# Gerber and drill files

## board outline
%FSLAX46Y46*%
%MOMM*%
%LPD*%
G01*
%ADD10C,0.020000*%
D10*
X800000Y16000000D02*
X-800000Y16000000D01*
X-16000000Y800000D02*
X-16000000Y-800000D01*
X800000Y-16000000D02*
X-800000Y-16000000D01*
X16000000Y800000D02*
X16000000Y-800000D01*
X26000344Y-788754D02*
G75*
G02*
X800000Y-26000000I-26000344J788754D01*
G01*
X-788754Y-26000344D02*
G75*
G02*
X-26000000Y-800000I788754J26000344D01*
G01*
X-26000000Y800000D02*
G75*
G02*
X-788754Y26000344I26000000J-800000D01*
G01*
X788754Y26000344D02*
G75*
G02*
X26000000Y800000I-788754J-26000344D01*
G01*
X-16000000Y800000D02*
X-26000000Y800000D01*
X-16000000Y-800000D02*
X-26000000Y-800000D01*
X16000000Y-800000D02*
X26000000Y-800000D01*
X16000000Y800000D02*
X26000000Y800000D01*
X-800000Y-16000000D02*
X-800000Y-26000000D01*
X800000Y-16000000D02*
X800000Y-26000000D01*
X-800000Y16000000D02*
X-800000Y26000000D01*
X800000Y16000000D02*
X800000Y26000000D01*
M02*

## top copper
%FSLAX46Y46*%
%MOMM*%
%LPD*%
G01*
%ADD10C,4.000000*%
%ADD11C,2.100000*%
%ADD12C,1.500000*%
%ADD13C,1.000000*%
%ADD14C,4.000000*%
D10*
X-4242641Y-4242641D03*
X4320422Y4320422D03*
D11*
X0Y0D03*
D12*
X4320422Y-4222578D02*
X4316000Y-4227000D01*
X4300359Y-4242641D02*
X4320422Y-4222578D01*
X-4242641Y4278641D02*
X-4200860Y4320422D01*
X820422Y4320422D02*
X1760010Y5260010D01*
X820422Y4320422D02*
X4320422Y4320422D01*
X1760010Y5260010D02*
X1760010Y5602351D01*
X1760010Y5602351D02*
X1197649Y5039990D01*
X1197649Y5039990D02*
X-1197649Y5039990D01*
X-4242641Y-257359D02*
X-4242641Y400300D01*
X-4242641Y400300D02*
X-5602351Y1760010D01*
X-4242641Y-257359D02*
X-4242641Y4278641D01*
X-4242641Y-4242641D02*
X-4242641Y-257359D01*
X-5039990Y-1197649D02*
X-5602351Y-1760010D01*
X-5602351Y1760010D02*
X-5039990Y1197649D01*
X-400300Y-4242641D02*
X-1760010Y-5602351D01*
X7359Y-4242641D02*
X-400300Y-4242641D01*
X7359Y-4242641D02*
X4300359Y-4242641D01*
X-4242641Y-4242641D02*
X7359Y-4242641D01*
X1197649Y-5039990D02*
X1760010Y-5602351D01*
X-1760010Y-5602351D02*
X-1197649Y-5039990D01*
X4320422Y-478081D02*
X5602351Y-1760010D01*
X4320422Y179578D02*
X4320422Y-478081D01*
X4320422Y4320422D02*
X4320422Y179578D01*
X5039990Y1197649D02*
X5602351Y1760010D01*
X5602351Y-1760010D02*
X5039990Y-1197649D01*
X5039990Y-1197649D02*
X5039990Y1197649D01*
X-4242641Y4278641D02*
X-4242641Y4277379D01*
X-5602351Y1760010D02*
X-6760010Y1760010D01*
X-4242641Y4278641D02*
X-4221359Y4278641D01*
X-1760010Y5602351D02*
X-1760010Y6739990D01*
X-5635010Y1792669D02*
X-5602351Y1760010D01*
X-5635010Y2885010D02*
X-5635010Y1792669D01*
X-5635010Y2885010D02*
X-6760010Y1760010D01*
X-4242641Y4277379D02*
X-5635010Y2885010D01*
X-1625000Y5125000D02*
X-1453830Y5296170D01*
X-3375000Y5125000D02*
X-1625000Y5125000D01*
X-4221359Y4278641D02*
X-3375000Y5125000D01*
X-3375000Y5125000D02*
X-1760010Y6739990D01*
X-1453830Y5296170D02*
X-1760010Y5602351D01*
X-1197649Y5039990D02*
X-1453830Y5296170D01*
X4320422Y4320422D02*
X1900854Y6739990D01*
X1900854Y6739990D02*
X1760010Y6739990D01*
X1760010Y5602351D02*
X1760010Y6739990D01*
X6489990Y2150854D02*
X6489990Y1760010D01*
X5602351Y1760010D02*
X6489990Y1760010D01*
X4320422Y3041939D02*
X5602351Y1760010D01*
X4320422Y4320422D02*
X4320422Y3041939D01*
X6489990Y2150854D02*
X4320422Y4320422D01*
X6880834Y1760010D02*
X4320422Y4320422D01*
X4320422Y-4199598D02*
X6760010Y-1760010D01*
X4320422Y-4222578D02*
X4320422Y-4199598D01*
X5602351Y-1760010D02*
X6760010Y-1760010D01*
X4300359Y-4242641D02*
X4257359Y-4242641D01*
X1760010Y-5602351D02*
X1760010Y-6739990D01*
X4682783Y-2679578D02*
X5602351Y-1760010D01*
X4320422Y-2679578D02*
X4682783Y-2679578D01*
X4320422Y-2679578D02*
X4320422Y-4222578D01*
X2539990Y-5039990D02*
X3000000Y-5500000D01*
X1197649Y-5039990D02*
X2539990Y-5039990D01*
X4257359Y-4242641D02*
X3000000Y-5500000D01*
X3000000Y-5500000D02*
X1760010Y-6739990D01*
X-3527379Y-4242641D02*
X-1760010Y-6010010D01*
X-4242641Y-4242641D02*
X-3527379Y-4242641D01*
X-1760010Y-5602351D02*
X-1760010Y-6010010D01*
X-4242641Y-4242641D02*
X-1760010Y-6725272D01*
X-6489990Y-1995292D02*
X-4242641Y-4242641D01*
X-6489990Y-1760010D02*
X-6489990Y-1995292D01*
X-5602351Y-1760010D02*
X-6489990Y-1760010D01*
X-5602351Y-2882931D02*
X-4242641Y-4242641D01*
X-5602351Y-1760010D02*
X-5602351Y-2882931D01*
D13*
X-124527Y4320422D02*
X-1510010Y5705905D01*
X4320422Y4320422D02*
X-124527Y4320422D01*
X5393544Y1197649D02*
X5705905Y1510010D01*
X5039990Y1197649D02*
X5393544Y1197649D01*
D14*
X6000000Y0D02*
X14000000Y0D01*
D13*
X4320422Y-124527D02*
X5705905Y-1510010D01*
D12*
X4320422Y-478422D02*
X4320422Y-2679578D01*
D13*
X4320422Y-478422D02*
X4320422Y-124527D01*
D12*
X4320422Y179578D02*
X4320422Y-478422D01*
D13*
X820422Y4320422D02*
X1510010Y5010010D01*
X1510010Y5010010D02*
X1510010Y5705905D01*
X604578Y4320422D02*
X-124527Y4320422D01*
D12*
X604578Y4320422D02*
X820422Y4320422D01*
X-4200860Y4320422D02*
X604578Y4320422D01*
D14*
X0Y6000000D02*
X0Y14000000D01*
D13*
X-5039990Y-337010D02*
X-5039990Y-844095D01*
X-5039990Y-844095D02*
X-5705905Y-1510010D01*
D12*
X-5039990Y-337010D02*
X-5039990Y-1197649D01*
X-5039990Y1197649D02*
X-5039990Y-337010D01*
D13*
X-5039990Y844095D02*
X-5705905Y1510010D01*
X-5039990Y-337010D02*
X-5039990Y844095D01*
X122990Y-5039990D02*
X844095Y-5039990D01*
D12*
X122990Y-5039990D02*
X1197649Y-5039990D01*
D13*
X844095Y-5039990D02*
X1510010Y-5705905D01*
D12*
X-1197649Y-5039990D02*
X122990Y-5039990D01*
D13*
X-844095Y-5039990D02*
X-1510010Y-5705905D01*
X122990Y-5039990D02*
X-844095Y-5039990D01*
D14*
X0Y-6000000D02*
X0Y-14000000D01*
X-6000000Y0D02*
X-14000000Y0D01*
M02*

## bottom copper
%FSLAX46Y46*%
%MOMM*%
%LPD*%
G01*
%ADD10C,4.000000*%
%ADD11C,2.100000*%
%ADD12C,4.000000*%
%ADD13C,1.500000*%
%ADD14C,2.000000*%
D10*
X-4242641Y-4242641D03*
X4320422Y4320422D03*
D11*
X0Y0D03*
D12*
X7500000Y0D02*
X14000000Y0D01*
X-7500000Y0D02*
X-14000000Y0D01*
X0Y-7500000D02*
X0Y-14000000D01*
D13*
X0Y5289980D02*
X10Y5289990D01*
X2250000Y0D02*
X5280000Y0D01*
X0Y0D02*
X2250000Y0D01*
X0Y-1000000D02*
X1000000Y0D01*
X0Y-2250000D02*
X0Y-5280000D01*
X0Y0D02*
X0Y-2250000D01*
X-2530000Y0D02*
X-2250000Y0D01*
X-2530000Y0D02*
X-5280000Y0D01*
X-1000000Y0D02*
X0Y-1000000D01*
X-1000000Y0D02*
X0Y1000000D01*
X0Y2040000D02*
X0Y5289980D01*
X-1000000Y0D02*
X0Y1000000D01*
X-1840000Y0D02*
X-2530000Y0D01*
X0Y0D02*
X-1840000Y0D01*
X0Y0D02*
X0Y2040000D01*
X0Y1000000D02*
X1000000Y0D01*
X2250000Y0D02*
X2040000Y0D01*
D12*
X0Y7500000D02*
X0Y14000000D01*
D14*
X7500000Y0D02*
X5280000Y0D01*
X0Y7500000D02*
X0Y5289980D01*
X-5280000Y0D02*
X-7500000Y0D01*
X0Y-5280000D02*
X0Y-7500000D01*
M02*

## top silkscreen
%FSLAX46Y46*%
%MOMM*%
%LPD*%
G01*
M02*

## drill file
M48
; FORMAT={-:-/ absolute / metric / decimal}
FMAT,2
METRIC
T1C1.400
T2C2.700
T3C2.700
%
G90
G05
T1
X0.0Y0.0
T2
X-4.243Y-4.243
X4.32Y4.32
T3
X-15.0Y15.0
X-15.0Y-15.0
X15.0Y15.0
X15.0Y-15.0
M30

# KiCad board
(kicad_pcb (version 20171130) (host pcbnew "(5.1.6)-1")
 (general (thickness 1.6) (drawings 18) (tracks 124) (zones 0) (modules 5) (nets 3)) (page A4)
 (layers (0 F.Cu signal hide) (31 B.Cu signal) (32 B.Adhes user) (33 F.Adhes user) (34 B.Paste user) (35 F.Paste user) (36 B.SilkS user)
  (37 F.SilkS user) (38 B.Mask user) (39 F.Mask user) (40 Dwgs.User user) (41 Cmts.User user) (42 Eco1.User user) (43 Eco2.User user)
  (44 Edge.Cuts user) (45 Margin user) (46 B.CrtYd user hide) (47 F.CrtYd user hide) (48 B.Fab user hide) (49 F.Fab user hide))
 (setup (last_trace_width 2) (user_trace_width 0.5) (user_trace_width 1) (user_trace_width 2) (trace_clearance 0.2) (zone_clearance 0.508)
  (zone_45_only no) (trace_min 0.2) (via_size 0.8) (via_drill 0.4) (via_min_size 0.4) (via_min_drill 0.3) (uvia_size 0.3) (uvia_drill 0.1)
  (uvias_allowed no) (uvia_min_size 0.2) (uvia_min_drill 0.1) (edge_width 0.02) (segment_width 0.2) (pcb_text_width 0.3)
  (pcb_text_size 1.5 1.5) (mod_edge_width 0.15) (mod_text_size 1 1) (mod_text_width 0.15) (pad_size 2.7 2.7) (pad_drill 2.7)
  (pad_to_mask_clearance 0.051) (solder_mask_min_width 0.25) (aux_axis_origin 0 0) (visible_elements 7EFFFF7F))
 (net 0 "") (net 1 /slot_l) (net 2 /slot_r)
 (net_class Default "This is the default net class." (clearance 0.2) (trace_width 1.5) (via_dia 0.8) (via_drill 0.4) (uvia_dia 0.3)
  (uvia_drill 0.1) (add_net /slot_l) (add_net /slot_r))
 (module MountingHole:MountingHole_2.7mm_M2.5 (layer F.Cu) (at -15 -15 90)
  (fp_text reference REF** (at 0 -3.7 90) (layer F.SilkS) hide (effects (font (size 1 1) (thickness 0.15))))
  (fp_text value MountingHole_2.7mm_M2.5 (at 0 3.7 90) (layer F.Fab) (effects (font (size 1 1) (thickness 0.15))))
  (pad 1 np_thru_hole circle (at 0 0 90) (size 2.7 2.7) (drill 2.7) (layers *.Cu *.Mask)))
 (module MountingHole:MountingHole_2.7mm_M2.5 (layer F.Cu) (at 15 -15)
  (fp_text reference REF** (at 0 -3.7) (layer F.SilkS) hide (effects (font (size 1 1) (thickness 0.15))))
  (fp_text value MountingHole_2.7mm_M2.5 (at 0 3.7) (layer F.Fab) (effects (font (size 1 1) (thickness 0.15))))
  (pad 1 np_thru_hole circle (at 0 0) (size 2.7 2.7) (drill 2.7) (layers *.Cu *.Mask)))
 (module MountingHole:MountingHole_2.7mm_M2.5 (layer F.Cu) (at 15 15)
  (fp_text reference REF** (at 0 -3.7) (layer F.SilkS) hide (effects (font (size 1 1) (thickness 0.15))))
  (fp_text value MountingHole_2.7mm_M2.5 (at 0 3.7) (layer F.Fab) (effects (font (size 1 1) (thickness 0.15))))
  (pad 1 np_thru_hole circle (at 0 0) (size 2.7 2.7) (drill 2.7) (layers *.Cu *.Mask)))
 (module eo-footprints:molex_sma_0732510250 (layer F.Cu) (at 0 0 45)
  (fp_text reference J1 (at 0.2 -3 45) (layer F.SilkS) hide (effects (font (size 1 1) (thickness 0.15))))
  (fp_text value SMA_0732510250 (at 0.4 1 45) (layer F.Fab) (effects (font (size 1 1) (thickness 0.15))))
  (pad 2 thru_hole circle (at -6 0 45) (size 4 4) (drill 2.7) (layers *.Cu *.Mask) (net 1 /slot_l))
  (pad 2 thru_hole circle (at 6.11 0 45) (size 4 4) (drill 2.7) (layers *.Cu *.Mask) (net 1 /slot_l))
  (pad 1 thru_hole circle (at 0 0 45) (size 2.1 2.1) (drill 1.4) (layers *.Cu *.Mask) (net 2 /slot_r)))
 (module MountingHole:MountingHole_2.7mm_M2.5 (layer F.Cu) (at -15 15)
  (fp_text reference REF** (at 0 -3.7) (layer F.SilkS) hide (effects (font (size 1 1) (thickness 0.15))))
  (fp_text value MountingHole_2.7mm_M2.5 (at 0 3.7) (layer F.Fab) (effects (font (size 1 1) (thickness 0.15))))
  (pad 1 np_thru_hole circle (at 0 0) (size 2.7 2.7) (drill 2.7) (layers *.Cu *.Mask)))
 (gr_line (start 0.8 -16) (end -0.8 -16) (layer Edge.Cuts) (width 0.02))
 (gr_line (start -16 -0.8) (end -16 0.8) (layer Edge.Cuts) (width 0.02))
 (gr_line (start 0.8 16) (end -0.8 16) (layer Edge.Cuts) (width 0.02))
 (gr_line (start 16 -0.8) (end 16 0.8) (layer Edge.Cuts) (width 0.02))
 (gr_arc (start 0 0) (end 0.8 26) (angle -86.5) (layer Edge.Cuts) (width 0.02))
 (gr_arc (start 0 0) (end -26 0.8) (angle -86.5) (layer Edge.Cuts) (width 0.02))
 (gr_arc (start 0 0) (end -26 -0.8) (angle 86.5) (layer Edge.Cuts) (width 0.02))
 (gr_arc (start 0 0) (end 26 -0.8) (angle -86.5) (layer Edge.Cuts) (width 0.02))
 (gr_line (start -16 -0.8) (end -26 -0.8) (layer Edge.Cuts) (width 0.02))
 (gr_line (start -16 0.8) (end -26 0.8) (layer Edge.Cuts) (width 0.02))
 (gr_line (start 16 0.8) (end 26 0.8) (layer Edge.Cuts) (width 0.02))
 (gr_line (start 16 -0.8) (end 26 -0.8) (layer Edge.Cuts) (width 0.02))
 (gr_line (start -0.8 16) (end -0.8 26) (layer Edge.Cuts) (width 0.02))
 (gr_line (start 0.8 16) (end 0.8 26) (layer Edge.Cuts) (width 0.02))
 (gr_line (start -0.8 -16) (end -0.8 -26) (layer Edge.Cuts) (width 0.02))
 (gr_line (start 0.8 -16) (end 0.8 -26) (layer Edge.Cuts) (width 0.02))
 (segment (start 7.5 0) (end 14 0) (width 4) (layer B.Cu) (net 2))
 (segment (start -7.5 0) (end -14 0) (width 4) (layer B.Cu) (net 2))
 (segment (start 0 7.5) (end 0 14) (width 4) (layer B.Cu) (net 2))
 (segment (start 0 -5.28998) (end 0.00001 -5.28999) (width 1.5) (layer B.Cu) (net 2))
 (segment (start 2.25 0) (end 5.28 0) (width 1.5) (layer B.Cu) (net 2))
 (segment (start 0 0) (end 2.25 0) (width 1.5) (layer B.Cu) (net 2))
 (segment (start 0 1) (end 1 0) (width 1.5) (layer B.Cu) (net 2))
 (segment (start 0 2.25) (end 0 5.28) (width 1.5) (layer B.Cu) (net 2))
 (segment (start 0 0) (end 0 2.25) (width 1.5) (layer B.Cu) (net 2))
 (segment (start -2.53 0) (end -2.25 0) (width 1.5) (layer B.Cu) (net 2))
 (segment (start -2.53 0) (end -5.28 0) (width 1.5) (layer B.Cu) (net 2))
 (segment (start -1 0) (end 0 1) (width 1.5) (layer B.Cu) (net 2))
 (segment (start -1 0) (end 0 -1) (width 1.5) (layer B.Cu) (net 2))
 (segment (start 0 -2.04) (end 0 -5.28998) (width 1.5) (layer B.Cu) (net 2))
 (segment (start -1 0) (end 0 -1) (width 1.5) (layer B.Cu) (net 2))
 (segment (start -1.84 0) (end -2.53 0) (width 1.5) (layer B.Cu) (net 2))
 (segment (start 0 0) (end -1.84 0) (width 1.5) (layer B.Cu) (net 2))
 (segment (start 0 0) (end 0 -2.04) (width 1.5) (layer B.Cu) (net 2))
 (segment (start 0 -1) (end 1 0) (width 1.5) (layer B.Cu) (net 2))
 (segment (start 2.25 0) (end 2.04 0) (width 1.5) (layer B.Cu) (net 2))
 (segment (start 0 -7.5) (end 0 -14) (width 4) (layer B.Cu) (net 2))
 (segment (start 7.5 0) (end 5.28 0) (width 2) (layer B.Cu) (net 2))
 (segment (start 0 -7.5) (end 0 -5.28998) (width 2) (layer B.Cu) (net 2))
 (segment (start -5.28 0) (end -7.5 0) (width 2) (layer B.Cu) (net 2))
 (segment (start 0 5.28) (end 0 7.5) (width 2) (layer B.Cu) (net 2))
 (segment (start 4.320422 4.222578) (end 4.316 4.227) (width 1.5) (layer F.Cu) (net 1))
 (segment (start 4.300359 4.242641) (end 4.320422 4.222578) (width 1.5) (layer F.Cu) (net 1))
 (segment (start -4.242641 -4.278641) (end -4.20086 -4.320422) (width 1.5) (layer F.Cu) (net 1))
 (segment (start 0.820422 -4.320422) (end 1.76001 -5.26001) (width 1.5) (layer F.Cu) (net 1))
 (segment (start 0.820422 -4.320422) (end 4.320422 -4.320422) (width 1.5) (layer F.Cu) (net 1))
 (segment (start 1.76001 -5.26001) (end 1.76001 -5.602351) (width 1.5) (layer F.Cu) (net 1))
 (segment (start 1.76001 -5.602351) (end 1.197649 -5.03999) (width 1.5) (layer F.Cu) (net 1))
 (segment (start 1.197649 -5.03999) (end -1.197649 -5.03999) (width 1.5) (layer F.Cu) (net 1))
 (segment (start -4.242641 0.257359) (end -4.242641 -0.4003) (width 1.5) (layer F.Cu) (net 1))
 (segment (start -4.242641 -0.4003) (end -5.602351 -1.76001) (width 1.5) (layer F.Cu) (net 1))
 (segment (start -4.242641 0.257359) (end -4.242641 -4.278641) (width 1.5) (layer F.Cu) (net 1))
 (segment (start -4.242641 4.242641) (end -4.242641 0.257359) (width 1.5) (layer F.Cu) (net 1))
 (segment (start -5.03999 1.197649) (end -5.602351 1.76001) (width 1.5) (layer F.Cu) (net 1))
 (segment (start -5.602351 -1.76001) (end -5.03999 -1.197649) (width 1.5) (layer F.Cu) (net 1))
 (segment (start -0.4003 4.242641) (end -1.76001 5.602351) (width 1.5) (layer F.Cu) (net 1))
 (segment (start 0.007359 4.242641) (end -0.4003 4.242641) (width 1.5) (layer F.Cu) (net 1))
 (segment (start 0.007359 4.242641) (end 4.300359 4.242641) (width 1.5) (layer F.Cu) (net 1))
 (segment (start -4.242641 4.242641) (end 0.007359 4.242641) (width 1.5) (layer F.Cu) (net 1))
 (segment (start 1.197649 5.03999) (end 1.76001 5.602351) (width 1.5) (layer F.Cu) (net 1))
 (segment (start -1.76001 5.602351) (end -1.197649 5.03999) (width 1.5) (layer F.Cu) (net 1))
 (segment (start 4.320422 0.478081) (end 5.602351 1.76001) (width 1.5) (layer F.Cu) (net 1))
 (segment (start 4.320422 -0.179578) (end 4.320422 0.478081) (width 1.5) (layer F.Cu) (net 1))
 (segment (start 4.320422 -4.320422) (end 4.320422 -0.179578) (width 1.5) (layer F.Cu) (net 1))
 (segment (start 5.03999 -1.197649) (end 5.602351 -1.76001) (width 1.5) (layer F.Cu) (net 1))
 (segment (start 5.602351 1.76001) (end 5.03999 1.197649) (width 1.5) (layer F.Cu) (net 1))
 (segment (start 5.03999 1.197649) (end 5.03999 -1.197649) (width 1.5) (layer F.Cu) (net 1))
 (segment (start -4.242641 -4.278641) (end -4.242641 -4.277379) (width 1.5) (layer F.Cu) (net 1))
 (segment (start -5.602351 -1.76001) (end -6.76001 -1.76001) (width 1.5) (layer F.Cu) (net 1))
 (segment (start -4.242641 -4.278641) (end -4.221359 -4.278641) (width 1.5) (layer F.Cu) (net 1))
 (segment (start -1.76001 -5.602351) (end -1.76001 -6.73999) (width 1.5) (layer F.Cu) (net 1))
 (segment (start -5.63501 -1.792669) (end -5.602351 -1.76001) (width 1.5) (layer F.Cu) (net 1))
 (segment (start -5.63501 -2.88501) (end -5.63501 -1.792669) (width 1.5) (layer F.Cu) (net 1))
 (segment (start -5.63501 -2.88501) (end -6.76001 -1.76001) (width 1.5) (layer F.Cu) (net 1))
 (segment (start -4.242641 -4.277379) (end -5.63501 -2.88501) (width 1.5) (layer F.Cu) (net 1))
 (segment (start -1.625 -5.125) (end -1.45383 -5.29617) (width 1.5) (layer F.Cu) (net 1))
 (segment (start -3.375 -5.125) (end -1.625 -5.125) (width 1.5) (layer F.Cu) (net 1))
 (segment (start -4.221359 -4.278641) (end -3.375 -5.125) (width 1.5) (layer F.Cu) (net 1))
 (segment (start -3.375 -5.125) (end -1.76001 -6.73999) (width 1.5) (layer F.Cu) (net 1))
 (segment (start -1.45383 -5.29617) (end -1.76001 -5.602351) (width 1.5) (layer F.Cu) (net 1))
 (segment (start -1.197649 -5.03999) (end -1.45383 -5.29617) (width 1.5) (layer F.Cu) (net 1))
 (segment (start 4.320422 -4.320422) (end 1.900854 -6.73999) (width 1.5) (layer F.Cu) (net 1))
 (segment (start 1.900854 -6.73999) (end 1.76001 -6.73999) (width 1.5) (layer F.Cu) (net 1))
 (segment (start 1.76001 -5.602351) (end 1.76001 -6.73999) (width 1.5) (layer F.Cu) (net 1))
 (segment (start 6.48999 -2.150854) (end 6.48999 -1.76001) (width 1.5) (layer F.Cu) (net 1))
 (segment (start 5.602351 -1.76001) (end 6.48999 -1.76001) (width 1.5) (layer F.Cu) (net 1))
 (segment (start 4.320422 -3.041939) (end 5.602351 -1.76001) (width 1.5) (layer F.Cu) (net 1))
 (segment (start 4.320422 -4.320422) (end 4.320422 -3.041939) (width 1.5) (layer F.Cu) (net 1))
 (segment (start 6.48999 -2.150854) (end 4.320422 -4.320422) (width 1.5) (layer F.Cu) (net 1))
 (segment (start 6.880834 -1.76001) (end 4.320422 -4.320422) (width 1.5) (layer F.Cu) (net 1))
 (segment (start 4.320422 4.199598) (end 6.76001 1.76001) (width 1.5) (layer F.Cu) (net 1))
 (segment (start 4.320422 4.222578) (end 4.320422 4.199598) (width 1.5) (layer F.Cu) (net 1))
 (segment (start 5.602351 1.76001) (end 6.76001 1.76001) (width 1.5) (layer F.Cu) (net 1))
 (segment (start 4.300359 4.242641) (end 4.257359 4.242641) (width 1.5) (layer F.Cu) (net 1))
 (segment (start 1.76001 5.602351) (end 1.76001 6.73999) (width 1.5) (layer F.Cu) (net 1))
 (segment (start 4.682783 2.679578) (end 5.602351 1.76001) (width 1.5) (layer F.Cu) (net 1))
 (segment (start 4.320422 2.679578) (end 4.682783 2.679578) (width 1.5) (layer F.Cu) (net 1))
 (segment (start 4.320422 2.679578) (end 4.320422 4.222578) (width 1.5) (layer F.Cu) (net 1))
 (segment (start 2.53999 5.03999) (end 3 5.5) (width 1.5) (layer F.Cu) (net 1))
 (segment (start 1.197649 5.03999) (end 2.53999 5.03999) (width 1.5) (layer F.Cu) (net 1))
 (segment (start 4.257359 4.242641) (end 3 5.5) (width 1.5) (layer F.Cu) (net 1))
 (segment (start 3 5.5) (end 1.76001 6.73999) (width 1.5) (layer F.Cu) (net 1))
 (segment (start -3.527379 4.242641) (end -1.76001 6.01001) (width 1.5) (layer F.Cu) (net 1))
 (segment (start -4.242641 4.242641) (end -3.527379 4.242641) (width 1.5) (layer F.Cu) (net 1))
 (segment (start -1.76001 5.602351) (end -1.76001 6.01001) (width 1.5) (layer F.Cu) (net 1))
 (segment (start -4.242641 4.242641) (end -1.76001 6.725272) (width 1.5) (layer F.Cu) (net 1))
 (segment (start -6.48999 1.995292) (end -4.242641 4.242641) (width 1.5) (layer F.Cu) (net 1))
 (segment (start -6.48999 1.76001) (end -6.48999 1.995292) (width 1.5) (layer F.Cu) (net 1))
 (segment (start -5.602351 1.76001) (end -6.48999 1.76001) (width 1.5) (layer F.Cu) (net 1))
 (segment (start -5.602351 2.882931) (end -4.242641 4.242641) (width 1.5) (layer F.Cu) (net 1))
 (segment (start -5.602351 1.76001) (end -5.602351 2.882931) (width 1.5) (layer F.Cu) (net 1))
 (segment (start -0.124527 -4.320422) (end -1.51001 -5.705905) (width 1) (layer F.Cu) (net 1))
 (segment (start 4.320422 -4.320422) (end -0.124527 -4.320422) (width 1) (layer F.Cu) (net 1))
 (segment (start 5.393544 -1.197649) (end 5.705905 -1.51001) (width 1) (layer F.Cu) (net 1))
 (segment (start 5.03999 -1.197649) (end 5.393544 -1.197649) (width 1) (layer F.Cu) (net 1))
 (segment (start 6 0) (end 14 0) (width 4) (layer F.Cu) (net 1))
 (segment (start 4.320422 0.124527) (end 5.705905 1.51001) (width 1) (layer F.Cu) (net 1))
 (segment (start 4.320422 0.478422) (end 4.320422 2.679578) (width 1.5) (layer F.Cu) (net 1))
 (segment (start 4.320422 0.478422) (end 4.320422 0.124527) (width 1) (layer F.Cu) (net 1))
 (segment (start 4.320422 -0.179578) (end 4.320422 0.478422) (width 1.5) (layer F.Cu) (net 1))
 (segment (start 0.820422 -4.320422) (end 1.51001 -5.01001) (width 1) (layer F.Cu) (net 1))
 (segment (start 1.51001 -5.01001) (end 1.51001 -5.705905) (width 1) (layer F.Cu) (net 1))
 (segment (start 0.604578 -4.320422) (end -0.124527 -4.320422) (width 1) (layer F.Cu) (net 1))
 (segment (start 0.604578 -4.320422) (end 0.820422 -4.320422) (width 1.5) (layer F.Cu) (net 1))
 (segment (start -4.20086 -4.320422) (end 0.604578 -4.320422) (width 1.5) (layer F.Cu) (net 1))
 (segment (start 0 -6) (end 0 -14) (width 4) (layer F.Cu) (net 1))
 (segment (start -5.03999 0.33701) (end -5.03999 0.844095) (width 1) (layer F.Cu) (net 1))
 (segment (start -5.03999 0.844095) (end -5.705905 1.51001) (width 1) (layer F.Cu) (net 1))
 (segment (start -5.03999 0.33701) (end -5.03999 1.197649) (width 1.5) (layer F.Cu) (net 1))
 (segment (start -5.03999 -1.197649) (end -5.03999 0.33701) (width 1.5) (layer F.Cu) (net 1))
 (segment (start -5.03999 -0.844095) (end -5.705905 -1.51001) (width 1) (layer F.Cu) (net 1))
 (segment (start -5.03999 0.33701) (end -5.03999 -0.844095) (width 1) (layer F.Cu) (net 1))
 (segment (start 0.12299 5.03999) (end 0.844095 5.03999) (width 1) (layer F.Cu) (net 1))
 (segment (start 0.12299 5.03999) (end 1.197649 5.03999) (width 1.5) (layer F.Cu) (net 1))
 (segment (start 0.844095 5.03999) (end 1.51001 5.705905) (width 1) (layer F.Cu) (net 1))
 (segment (start -1.197649 5.03999) (end 0.12299 5.03999) (width 1.5) (layer F.Cu) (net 1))
 (segment (start -0.844095 5.03999) (end -1.51001 5.705905) (width 1) (layer F.Cu) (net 1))
 (segment (start 0.12299 5.03999) (end -0.844095 5.03999) (width 1) (layer F.Cu) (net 1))
 (segment (start 0 6) (end 0 14) (width 4) (layer F.Cu) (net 1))
 (segment (start -6 0) (end -14 0) (width 4) (layer F.Cu) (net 1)))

